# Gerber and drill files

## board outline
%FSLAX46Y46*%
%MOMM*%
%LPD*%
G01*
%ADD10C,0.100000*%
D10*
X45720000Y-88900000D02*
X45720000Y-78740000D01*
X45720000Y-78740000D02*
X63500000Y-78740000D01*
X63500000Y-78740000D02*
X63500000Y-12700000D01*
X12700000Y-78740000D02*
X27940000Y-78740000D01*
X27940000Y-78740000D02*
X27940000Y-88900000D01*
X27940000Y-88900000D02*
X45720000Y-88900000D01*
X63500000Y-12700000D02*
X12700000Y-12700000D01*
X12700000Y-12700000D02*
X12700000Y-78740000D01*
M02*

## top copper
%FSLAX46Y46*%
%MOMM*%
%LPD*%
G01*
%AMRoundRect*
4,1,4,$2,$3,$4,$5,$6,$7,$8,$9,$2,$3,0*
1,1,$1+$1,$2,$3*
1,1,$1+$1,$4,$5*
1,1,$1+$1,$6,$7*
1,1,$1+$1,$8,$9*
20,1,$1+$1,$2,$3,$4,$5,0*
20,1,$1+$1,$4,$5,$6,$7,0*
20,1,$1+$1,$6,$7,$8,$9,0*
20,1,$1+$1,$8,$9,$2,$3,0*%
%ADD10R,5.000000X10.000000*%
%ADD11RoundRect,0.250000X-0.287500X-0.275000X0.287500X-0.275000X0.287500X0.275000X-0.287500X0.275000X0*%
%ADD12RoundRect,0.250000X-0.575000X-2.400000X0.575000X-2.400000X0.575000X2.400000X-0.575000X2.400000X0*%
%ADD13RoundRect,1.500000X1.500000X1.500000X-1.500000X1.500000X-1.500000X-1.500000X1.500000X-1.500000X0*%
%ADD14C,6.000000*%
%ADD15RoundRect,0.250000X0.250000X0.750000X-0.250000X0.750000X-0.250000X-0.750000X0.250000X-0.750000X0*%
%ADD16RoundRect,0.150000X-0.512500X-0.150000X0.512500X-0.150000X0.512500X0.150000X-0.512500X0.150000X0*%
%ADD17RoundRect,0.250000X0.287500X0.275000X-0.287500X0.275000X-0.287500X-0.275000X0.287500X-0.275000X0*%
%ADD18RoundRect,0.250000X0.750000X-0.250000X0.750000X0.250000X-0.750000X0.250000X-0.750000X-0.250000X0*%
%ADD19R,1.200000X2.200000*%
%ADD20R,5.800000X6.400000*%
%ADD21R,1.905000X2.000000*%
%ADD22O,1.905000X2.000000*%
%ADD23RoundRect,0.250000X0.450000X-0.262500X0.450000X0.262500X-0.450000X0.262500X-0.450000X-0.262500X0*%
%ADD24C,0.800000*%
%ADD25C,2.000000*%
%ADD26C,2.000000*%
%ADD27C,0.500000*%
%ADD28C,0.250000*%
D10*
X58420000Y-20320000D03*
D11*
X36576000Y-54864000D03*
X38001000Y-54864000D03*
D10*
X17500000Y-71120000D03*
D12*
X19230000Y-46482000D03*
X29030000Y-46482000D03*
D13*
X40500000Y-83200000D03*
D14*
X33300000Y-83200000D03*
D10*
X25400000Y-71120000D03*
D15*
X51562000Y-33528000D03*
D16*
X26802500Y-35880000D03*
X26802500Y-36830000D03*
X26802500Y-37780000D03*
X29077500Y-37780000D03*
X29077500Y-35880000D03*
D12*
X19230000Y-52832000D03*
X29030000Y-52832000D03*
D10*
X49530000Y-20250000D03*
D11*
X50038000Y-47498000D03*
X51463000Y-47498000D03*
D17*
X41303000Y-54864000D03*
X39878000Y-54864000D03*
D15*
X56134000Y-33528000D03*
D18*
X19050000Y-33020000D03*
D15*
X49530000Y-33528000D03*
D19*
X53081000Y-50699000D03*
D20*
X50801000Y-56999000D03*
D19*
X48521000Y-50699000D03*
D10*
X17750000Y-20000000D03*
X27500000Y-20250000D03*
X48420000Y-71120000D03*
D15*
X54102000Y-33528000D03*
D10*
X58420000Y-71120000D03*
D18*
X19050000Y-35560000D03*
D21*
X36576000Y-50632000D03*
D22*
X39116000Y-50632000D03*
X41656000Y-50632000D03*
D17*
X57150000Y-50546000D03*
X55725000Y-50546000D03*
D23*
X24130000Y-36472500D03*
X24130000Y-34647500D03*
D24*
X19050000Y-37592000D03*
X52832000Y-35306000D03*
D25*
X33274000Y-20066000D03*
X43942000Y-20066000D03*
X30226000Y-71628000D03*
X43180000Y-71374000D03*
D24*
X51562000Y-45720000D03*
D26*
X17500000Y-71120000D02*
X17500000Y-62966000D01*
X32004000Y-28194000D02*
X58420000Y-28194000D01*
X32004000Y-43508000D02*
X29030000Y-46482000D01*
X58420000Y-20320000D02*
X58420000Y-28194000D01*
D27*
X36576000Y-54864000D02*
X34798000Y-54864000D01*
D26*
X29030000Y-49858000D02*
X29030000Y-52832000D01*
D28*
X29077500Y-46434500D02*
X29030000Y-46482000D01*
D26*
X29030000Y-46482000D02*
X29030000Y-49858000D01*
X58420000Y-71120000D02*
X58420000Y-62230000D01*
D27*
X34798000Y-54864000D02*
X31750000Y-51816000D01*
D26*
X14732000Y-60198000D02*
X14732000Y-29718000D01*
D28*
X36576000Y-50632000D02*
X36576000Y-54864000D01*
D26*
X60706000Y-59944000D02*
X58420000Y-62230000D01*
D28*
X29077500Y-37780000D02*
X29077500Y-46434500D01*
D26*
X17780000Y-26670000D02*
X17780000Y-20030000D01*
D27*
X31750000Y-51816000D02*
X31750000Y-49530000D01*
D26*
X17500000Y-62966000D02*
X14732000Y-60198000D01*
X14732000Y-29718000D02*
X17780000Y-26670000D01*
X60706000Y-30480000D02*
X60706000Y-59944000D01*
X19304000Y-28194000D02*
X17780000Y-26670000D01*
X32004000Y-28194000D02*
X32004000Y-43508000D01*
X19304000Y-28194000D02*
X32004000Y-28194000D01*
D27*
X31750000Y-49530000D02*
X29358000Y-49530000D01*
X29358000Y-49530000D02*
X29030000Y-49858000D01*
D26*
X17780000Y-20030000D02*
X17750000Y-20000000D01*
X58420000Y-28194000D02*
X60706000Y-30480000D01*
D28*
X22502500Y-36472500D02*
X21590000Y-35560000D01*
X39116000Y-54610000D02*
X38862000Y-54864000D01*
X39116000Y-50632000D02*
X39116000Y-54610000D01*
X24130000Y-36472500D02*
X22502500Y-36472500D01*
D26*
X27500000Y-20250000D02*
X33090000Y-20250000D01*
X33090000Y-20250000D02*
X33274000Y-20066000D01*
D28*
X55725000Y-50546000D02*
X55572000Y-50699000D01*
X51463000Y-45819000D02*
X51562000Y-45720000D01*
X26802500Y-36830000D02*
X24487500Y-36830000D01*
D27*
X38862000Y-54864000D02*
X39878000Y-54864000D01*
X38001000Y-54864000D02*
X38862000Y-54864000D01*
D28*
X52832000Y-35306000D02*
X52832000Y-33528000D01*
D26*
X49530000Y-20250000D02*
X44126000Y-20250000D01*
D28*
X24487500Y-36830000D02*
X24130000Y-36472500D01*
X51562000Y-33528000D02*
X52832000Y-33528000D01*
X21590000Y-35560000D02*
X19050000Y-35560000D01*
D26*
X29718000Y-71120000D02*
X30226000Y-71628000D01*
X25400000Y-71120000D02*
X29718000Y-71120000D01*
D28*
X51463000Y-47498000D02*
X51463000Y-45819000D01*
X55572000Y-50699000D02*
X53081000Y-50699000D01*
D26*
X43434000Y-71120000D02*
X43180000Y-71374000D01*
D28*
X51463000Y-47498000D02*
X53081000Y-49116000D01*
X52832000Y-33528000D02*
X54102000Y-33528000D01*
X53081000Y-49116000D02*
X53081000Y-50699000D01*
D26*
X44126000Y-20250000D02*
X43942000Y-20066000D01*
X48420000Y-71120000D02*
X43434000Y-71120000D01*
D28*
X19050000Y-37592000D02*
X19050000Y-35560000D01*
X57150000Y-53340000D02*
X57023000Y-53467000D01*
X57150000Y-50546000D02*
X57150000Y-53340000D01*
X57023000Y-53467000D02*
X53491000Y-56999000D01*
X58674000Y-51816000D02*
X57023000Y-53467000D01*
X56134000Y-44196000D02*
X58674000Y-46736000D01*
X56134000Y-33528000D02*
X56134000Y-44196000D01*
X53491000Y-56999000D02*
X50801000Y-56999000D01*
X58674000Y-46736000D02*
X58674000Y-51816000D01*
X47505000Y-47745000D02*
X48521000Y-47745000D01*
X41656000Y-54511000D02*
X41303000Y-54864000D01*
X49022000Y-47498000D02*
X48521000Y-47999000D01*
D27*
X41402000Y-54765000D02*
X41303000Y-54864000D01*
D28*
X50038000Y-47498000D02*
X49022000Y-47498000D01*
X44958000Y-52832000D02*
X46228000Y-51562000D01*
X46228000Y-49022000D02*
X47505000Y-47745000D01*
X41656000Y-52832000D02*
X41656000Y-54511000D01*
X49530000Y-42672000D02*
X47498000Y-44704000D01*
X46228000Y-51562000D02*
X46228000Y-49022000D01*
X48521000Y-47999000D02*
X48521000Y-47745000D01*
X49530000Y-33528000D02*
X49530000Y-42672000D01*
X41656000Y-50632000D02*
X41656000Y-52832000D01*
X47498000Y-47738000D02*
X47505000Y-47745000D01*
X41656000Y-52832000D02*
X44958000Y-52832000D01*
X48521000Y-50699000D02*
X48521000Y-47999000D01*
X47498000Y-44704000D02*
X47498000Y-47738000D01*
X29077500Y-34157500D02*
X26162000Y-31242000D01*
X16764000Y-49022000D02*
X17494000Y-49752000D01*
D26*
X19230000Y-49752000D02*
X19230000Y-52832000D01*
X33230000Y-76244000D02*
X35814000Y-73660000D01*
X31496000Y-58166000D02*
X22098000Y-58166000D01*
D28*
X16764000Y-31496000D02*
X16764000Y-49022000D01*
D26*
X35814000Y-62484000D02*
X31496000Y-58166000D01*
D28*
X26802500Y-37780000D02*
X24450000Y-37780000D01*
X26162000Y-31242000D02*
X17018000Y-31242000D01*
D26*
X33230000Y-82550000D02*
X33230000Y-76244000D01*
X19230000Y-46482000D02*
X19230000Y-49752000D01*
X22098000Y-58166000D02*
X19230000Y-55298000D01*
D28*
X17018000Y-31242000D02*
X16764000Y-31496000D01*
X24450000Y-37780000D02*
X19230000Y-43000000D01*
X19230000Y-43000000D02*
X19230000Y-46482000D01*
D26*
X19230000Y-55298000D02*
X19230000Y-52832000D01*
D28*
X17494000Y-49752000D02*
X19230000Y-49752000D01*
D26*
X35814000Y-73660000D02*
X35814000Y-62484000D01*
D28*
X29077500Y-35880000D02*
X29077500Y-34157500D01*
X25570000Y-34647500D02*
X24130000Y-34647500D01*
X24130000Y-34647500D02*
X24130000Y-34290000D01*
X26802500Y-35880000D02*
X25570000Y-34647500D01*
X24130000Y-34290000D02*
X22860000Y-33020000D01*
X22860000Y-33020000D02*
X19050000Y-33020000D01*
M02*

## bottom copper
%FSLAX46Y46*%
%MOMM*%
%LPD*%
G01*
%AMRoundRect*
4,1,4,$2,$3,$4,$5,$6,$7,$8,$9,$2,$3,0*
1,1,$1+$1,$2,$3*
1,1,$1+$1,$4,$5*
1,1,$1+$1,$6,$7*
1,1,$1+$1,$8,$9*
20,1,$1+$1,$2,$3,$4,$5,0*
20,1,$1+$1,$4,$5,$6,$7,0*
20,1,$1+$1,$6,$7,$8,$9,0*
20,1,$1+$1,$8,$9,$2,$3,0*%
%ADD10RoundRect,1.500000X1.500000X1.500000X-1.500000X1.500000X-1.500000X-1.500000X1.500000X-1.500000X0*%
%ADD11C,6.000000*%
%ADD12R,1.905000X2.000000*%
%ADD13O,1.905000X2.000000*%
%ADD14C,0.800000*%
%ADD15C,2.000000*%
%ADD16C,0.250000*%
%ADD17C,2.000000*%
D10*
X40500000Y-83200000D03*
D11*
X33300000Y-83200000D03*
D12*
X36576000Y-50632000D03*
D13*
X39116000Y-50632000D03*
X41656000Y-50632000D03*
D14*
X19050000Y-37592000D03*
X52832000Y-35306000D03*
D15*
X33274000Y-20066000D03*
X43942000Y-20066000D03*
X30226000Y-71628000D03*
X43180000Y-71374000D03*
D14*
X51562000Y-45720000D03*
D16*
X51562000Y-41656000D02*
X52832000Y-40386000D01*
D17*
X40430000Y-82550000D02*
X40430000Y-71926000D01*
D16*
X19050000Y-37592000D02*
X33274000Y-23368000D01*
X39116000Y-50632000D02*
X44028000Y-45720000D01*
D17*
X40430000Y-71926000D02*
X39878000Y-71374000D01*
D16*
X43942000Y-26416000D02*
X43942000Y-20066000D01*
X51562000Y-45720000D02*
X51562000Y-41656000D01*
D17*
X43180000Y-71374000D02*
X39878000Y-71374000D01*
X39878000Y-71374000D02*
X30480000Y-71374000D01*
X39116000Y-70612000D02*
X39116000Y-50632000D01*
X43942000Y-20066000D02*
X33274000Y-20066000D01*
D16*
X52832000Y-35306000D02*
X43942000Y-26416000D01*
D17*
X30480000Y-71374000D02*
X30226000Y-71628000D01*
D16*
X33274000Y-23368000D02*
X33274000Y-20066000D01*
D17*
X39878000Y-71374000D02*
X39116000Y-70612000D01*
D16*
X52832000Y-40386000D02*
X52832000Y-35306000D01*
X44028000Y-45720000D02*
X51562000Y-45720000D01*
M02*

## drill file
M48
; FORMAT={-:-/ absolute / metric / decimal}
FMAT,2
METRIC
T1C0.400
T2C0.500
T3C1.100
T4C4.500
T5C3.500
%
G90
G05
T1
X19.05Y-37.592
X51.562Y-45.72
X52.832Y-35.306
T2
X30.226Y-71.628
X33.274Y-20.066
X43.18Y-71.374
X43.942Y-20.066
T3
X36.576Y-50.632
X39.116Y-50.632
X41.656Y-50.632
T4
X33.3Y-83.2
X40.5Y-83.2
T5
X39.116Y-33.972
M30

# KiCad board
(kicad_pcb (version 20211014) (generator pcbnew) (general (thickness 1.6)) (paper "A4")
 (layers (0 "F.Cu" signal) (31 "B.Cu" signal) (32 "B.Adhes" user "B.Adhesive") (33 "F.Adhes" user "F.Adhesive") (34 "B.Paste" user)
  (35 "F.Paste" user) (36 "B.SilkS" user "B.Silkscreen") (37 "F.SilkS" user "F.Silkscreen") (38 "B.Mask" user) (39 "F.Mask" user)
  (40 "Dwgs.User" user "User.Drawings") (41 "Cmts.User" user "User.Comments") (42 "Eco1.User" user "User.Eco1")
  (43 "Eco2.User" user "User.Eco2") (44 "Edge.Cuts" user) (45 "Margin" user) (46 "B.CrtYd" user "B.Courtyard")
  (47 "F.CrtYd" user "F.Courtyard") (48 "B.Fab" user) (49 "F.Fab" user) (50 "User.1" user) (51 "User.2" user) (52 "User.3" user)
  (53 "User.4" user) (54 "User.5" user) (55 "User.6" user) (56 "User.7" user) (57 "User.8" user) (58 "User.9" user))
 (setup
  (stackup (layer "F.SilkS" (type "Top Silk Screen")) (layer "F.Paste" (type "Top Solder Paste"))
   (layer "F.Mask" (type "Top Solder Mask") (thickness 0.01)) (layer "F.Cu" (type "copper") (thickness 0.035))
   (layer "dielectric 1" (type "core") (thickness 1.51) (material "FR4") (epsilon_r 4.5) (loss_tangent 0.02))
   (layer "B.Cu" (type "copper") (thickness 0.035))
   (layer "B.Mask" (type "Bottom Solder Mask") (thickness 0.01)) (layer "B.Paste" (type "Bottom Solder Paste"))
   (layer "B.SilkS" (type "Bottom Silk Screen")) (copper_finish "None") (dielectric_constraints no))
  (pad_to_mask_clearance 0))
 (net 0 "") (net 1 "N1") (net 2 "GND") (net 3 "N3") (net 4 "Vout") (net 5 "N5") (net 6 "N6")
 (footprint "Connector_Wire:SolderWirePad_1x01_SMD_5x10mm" (layer "F.Cu") (at 58.42 20.32)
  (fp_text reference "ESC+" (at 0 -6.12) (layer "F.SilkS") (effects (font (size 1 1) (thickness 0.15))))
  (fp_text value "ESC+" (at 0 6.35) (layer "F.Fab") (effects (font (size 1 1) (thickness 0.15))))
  (pad "1" smd rect (at 0 0) (size 5 10) (layers "F.Cu" "F.Paste" "F.Mask") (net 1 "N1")))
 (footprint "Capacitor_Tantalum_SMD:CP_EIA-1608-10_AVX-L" (layer "F.Cu") (at 37.2885 54.864)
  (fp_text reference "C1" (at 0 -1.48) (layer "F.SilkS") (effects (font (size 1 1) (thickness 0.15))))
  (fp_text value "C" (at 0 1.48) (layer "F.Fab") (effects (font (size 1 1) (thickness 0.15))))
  (pad "1" smd roundrect (at -0.7125 0) (size 1.075 1.05) (layers "F.Cu" "F.Paste" "F.Mask") (roundrect_rratio 0.238095) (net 1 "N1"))
  (pad "2" smd roundrect (at 0.7125 0) (size 1.075 1.05) (layers "F.Cu" "F.Paste" "F.Mask") (roundrect_rratio 0.238095) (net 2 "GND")))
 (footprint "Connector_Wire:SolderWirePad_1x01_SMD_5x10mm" (layer "F.Cu") (at 17.5 71.12)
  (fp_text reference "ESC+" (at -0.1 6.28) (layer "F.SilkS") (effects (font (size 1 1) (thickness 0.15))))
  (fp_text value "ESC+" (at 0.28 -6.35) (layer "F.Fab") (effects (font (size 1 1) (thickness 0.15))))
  (pad "1" smd rect (at 0 0) (size 5 10) (layers "F.Cu" "F.Paste" "F.Mask") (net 1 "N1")))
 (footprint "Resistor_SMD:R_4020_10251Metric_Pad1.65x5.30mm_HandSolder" (layer "F.Cu") (at 24.13 46.482)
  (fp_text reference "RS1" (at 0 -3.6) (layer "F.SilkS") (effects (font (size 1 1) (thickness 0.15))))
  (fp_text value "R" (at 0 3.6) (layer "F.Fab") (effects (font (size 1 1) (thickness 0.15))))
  (pad "1" smd roundrect (at -4.9 0) (size 1.65 5.3) (layers "F.Cu" "F.Paste" "F.Mask") (roundrect_rratio 0.151515) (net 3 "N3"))
  (pad "2" smd roundrect (at 4.9 0) (size 1.65 5.3) (layers "F.Cu" "F.Paste" "F.Mask") (roundrect_rratio 0.151515) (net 1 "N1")))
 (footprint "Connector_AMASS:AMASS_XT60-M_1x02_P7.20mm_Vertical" (layer "F.Cu") (at 40.5 83.2 180)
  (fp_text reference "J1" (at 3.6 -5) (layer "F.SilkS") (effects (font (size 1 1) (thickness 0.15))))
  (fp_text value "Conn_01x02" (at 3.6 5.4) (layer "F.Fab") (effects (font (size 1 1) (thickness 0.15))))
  (pad "1" thru_hole roundrect (at 0 0 180) (size 6 6) (drill 4.5) (layers *.Cu *.Mask) (roundrect_rratio 0.25) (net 2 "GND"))
  (pad "2" thru_hole circle (at 7.2 0 180) (size 6 6) (drill 4.5) (layers *.Cu *.Mask) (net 3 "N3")))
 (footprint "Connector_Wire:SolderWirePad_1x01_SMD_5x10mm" (layer "F.Cu") (at 25.4 71.12)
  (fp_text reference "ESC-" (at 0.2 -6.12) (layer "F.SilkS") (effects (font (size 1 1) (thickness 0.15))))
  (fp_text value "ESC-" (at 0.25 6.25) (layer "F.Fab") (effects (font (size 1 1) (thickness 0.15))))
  (pad "1" smd rect (at 0 0) (size 5 10) (layers "F.Cu" "F.Paste" "F.Mask") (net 2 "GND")))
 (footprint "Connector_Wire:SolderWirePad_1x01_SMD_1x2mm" (layer "F.Cu") (at 51.562 33.528 180)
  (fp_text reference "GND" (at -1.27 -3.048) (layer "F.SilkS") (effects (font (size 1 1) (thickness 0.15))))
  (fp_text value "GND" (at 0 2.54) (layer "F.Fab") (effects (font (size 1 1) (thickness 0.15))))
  (pad "1" smd roundrect (at 0 0 180) (size 1 2) (layers "F.Cu" "F.Paste" "F.Mask") (roundrect_rratio 0.25) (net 2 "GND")))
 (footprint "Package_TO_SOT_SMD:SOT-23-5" (layer "F.Cu") (at 27.94 36.83)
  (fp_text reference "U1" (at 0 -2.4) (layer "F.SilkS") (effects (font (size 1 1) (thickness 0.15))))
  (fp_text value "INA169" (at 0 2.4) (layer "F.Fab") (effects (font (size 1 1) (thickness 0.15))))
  (pad "1" smd roundrect (at -1.1375 -0.95) (size 1.325 0.6) (layers "F.Cu" "F.Paste" "F.Mask") (roundrect_rratio 0.25) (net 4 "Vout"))
  (pad "2" smd roundrect (at -1.1375 0) (size 1.325 0.6) (layers "F.Cu" "F.Paste" "F.Mask") (roundrect_rratio 0.25) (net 2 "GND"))
  (pad "3" smd roundrect (at -1.1375 0.95) (size 1.325 0.6) (layers "F.Cu" "F.Paste" "F.Mask") (roundrect_rratio 0.25) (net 3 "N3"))
  (pad "4" smd roundrect (at 1.1375 0.95) (size 1.325 0.6) (layers "F.Cu" "F.Paste" "F.Mask") (roundrect_rratio 0.25) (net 1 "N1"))
  (pad "5" smd roundrect (at 1.1375 -0.95) (size 1.325 0.6) (layers "F.Cu" "F.Paste" "F.Mask") (roundrect_rratio 0.25) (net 3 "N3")))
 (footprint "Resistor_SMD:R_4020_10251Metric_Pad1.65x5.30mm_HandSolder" (layer "F.Cu") (at 24.13 52.832)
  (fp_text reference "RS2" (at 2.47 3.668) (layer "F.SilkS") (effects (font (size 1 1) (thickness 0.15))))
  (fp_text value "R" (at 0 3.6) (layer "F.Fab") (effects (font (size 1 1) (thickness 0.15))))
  (pad "1" smd roundrect (at -4.9 0) (size 1.65 5.3) (layers "F.Cu" "F.Paste" "F.Mask") (roundrect_rratio 0.151515) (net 3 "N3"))
  (pad "2" smd roundrect (at 4.9 0) (size 1.65 5.3) (layers "F.Cu" "F.Paste" "F.Mask") (roundrect_rratio 0.151515) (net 1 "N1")))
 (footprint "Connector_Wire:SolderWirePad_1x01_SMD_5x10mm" (layer "F.Cu") (at 49.53 20.25)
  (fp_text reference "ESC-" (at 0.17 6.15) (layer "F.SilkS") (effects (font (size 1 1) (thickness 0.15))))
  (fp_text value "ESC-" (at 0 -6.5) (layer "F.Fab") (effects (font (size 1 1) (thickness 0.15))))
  (pad "1" smd rect (at 0 0) (size 5 10) (layers "F.Cu" "F.Paste" "F.Mask") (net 2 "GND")))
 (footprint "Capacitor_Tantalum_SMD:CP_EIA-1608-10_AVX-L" (layer "F.Cu") (at 50.7505 47.498)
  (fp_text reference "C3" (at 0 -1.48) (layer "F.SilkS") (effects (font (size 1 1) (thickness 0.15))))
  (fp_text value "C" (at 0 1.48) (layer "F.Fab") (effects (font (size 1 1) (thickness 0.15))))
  (pad "1" smd roundrect (at -0.7125 0) (size 1.075 1.05) (layers "F.Cu" "F.Paste" "F.Mask") (roundrect_rratio 0.238095) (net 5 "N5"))
  (pad "2" smd roundrect (at 0.7125 0) (size 1.075 1.05) (layers "F.Cu" "F.Paste" "F.Mask") (roundrect_rratio 0.238095) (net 2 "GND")))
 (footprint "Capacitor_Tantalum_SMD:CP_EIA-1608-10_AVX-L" (layer "F.Cu") (at 40.5905 54.864 180)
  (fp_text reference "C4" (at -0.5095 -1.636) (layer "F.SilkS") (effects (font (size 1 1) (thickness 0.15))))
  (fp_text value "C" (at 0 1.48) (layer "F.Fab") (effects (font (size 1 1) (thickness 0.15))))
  (pad "1" smd roundrect (at -0.7125 0 180) (size 1.075 1.05) (layers "F.Cu" "F.Paste" "F.Mask") (roundrect_rratio 0.238095) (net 5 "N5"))
  (pad "2" smd roundrect (at 0.7125 0 180) (size 1.075 1.05) (layers "F.Cu" "F.Paste" "F.Mask") (roundrect_rratio 0.238095) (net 2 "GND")))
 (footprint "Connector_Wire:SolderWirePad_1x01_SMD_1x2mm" (layer "F.Cu") (at 56.134 33.528 180)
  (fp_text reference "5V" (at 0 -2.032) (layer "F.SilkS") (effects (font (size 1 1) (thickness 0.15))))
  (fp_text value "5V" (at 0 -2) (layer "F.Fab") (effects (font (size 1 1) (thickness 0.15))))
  (pad "1" smd roundrect (at 0 0 180) (size 1 2) (layers "F.Cu" "F.Paste" "F.Mask") (roundrect_rratio 0.25) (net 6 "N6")))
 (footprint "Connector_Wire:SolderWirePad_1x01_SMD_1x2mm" (layer "F.Cu") (at 19.05 33.02 90)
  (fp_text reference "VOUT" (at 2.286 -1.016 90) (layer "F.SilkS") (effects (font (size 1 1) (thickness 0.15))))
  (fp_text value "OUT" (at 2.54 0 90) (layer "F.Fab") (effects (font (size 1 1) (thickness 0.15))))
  (pad "1" smd roundrect (at 0 0 90) (size 1 2) (layers "F.Cu" "F.Paste" "F.Mask") (roundrect_rratio 0.25) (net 4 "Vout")))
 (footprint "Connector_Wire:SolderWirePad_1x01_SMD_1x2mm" (layer "F.Cu") (at 49.53 33.528 180)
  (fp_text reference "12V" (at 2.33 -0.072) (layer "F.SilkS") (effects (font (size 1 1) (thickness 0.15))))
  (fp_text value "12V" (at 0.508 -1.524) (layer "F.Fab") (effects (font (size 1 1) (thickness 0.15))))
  (pad "1" smd roundrect (at 0 0 180) (size 1 2) (layers "F.Cu" "F.Paste" "F.Mask") (roundrect_rratio 0.25) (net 5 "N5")))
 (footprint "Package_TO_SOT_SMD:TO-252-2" (layer "F.Cu") (at 50.801 54.899 -90)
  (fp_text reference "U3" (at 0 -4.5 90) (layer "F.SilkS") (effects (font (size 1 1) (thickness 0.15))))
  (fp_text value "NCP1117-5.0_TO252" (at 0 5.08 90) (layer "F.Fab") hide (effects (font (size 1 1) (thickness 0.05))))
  (pad "" smd rect (at 0.425 1.525 270) (size 3.05 2.75) (layers "F.Paste"))
  (pad "" smd rect (at 3.775 1.525 270) (size 3.05 2.75) (layers "F.Paste"))
  (pad "" smd rect (at 3.775 -1.525 270) (size 3.05 2.75) (layers "F.Paste"))
  (pad "" smd rect (at 0.425 -1.525 270) (size 3.05 2.75) (layers "F.Paste"))
  (pad "1" smd rect (at -4.2 -2.28 270) (size 2.2 1.2) (layers "F.Cu" "F.Paste" "F.Mask") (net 2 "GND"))
  (pad "2" smd rect (at 2.1 0 270) (size 6.4 5.8) (layers "F.Cu" "F.Mask") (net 6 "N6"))
  (pad "3" smd rect (at -4.2 2.28 270) (size 2.2 1.2) (layers "F.Cu" "F.Paste" "F.Mask") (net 5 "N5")))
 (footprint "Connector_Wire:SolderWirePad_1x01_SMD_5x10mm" (layer "F.Cu") (at 17.75 20)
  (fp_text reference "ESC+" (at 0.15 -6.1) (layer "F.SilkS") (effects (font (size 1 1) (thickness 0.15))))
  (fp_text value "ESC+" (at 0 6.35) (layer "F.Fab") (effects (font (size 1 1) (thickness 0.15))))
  (pad "1" smd rect (at 0 0) (size 5 10) (layers "F.Cu" "F.Paste" "F.Mask") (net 1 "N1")))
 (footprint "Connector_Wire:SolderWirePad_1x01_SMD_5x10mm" (layer "F.Cu") (at 27.5 20.25)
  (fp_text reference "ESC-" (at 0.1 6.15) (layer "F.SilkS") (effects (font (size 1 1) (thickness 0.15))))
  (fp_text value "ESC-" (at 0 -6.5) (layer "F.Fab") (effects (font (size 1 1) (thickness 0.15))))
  (pad "1" smd rect (at 0 0) (size 5 10) (layers "F.Cu" "F.Paste" "F.Mask") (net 2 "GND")))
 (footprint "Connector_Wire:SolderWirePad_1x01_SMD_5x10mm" (layer "F.Cu") (at 48.42 71.12)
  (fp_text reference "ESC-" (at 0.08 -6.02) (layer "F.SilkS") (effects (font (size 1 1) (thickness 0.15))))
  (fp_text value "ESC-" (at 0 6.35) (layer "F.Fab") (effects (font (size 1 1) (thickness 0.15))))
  (pad "1" smd rect (at 0 0) (size 5 10) (layers "F.Cu" "F.Paste" "F.Mask") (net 2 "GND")))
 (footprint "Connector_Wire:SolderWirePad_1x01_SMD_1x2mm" (layer "F.Cu") (at 54.102 33.528 180)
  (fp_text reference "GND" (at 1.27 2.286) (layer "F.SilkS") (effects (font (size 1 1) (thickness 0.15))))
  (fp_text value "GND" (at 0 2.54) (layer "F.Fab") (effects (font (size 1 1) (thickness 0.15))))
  (pad "1" smd roundrect (at 0 0 180) (size 1 2) (layers "F.Cu" "F.Paste" "F.Mask") (roundrect_rratio 0.25) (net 2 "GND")))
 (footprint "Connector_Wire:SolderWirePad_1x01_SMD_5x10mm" (layer "F.Cu") (at 58.42 71.12)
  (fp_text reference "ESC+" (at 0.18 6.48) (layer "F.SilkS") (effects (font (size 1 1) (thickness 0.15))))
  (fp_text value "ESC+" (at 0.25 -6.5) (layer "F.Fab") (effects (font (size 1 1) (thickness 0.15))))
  (pad "1" smd rect (at 0 0) (size 5 10) (layers "F.Cu" "F.Paste" "F.Mask") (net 1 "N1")))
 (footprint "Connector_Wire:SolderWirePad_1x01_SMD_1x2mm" (layer "F.Cu") (at 19.05 35.56 90)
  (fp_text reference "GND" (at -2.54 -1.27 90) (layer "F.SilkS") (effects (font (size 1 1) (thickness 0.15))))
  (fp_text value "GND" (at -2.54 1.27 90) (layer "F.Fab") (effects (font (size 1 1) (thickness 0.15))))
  (pad "1" smd roundrect (at 0 0 90) (size 1 2) (layers "F.Cu" "F.Paste" "F.Mask") (roundrect_rratio 0.25) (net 2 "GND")))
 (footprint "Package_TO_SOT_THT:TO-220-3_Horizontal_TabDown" (layer "F.Cu") (at 36.576 50.632)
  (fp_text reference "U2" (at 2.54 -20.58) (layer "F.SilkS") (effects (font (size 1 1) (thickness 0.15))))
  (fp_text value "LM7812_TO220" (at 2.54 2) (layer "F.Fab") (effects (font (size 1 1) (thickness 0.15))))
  (pad "" np_thru_hole oval (at 2.54 -16.66) (size 3.5 3.5) (drill 3.5) (layers *.Cu *.Mask))
  (pad "1" thru_hole rect (at 0 0) (size 1.905 2) (drill 1.1) (layers *.Cu *.Mask) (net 1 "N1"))
  (pad "2" thru_hole oval (at 2.54 0) (size 1.905 2) (drill 1.1) (layers *.Cu *.Mask) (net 2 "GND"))
  (pad "3" thru_hole oval (at 5.08 0) (size 1.905 2) (drill 1.1) (layers *.Cu *.Mask) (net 5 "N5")))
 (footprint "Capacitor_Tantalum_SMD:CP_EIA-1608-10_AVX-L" (layer "F.Cu") (at 56.4375 50.546 180)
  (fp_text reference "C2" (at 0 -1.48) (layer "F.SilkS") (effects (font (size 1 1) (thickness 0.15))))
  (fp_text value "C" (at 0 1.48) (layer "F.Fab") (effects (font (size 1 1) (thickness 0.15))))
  (pad "1" smd roundrect (at -0.7125 0 180) (size 1.075 1.05) (layers "F.Cu" "F.Paste" "F.Mask") (roundrect_rratio 0.238095) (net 6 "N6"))
  (pad "2" smd roundrect (at 0.7125 0 180) (size 1.075 1.05) (layers "F.Cu" "F.Paste" "F.Mask") (roundrect_rratio 0.238095) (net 2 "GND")))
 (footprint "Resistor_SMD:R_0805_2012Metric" (layer "F.Cu") (at 24.13 35.56 90)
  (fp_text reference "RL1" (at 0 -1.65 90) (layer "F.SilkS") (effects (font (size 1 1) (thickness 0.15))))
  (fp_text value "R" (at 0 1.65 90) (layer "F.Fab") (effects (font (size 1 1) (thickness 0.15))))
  (pad "1" smd roundrect (at -0.9125 0 90) (size 1.025 1.4) (layers "F.Cu" "F.Paste" "F.Mask") (roundrect_rratio 0.243902) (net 2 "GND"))
  (pad "2" smd roundrect (at 0.9125 0 90) (size 1.025 1.4) (layers "F.Cu" "F.Paste" "F.Mask") (roundrect_rratio 0.243902) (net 4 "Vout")))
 (gr_line (start 45.72 88.9) (end 45.72 78.74) (layer "Edge.Cuts") (width 0.1))
 (gr_line (start 45.72 78.74) (end 63.5 78.74) (layer "Edge.Cuts") (width 0.1))
 (gr_line (start 63.5 78.74) (end 63.5 12.7) (layer "Edge.Cuts") (width 0.1))
 (gr_line (start 12.7 78.74) (end 27.94 78.74) (layer "Edge.Cuts") (width 0.1))
 (gr_line (start 27.94 78.74) (end 27.94 88.9) (layer "Edge.Cuts") (width 0.1))
 (gr_line (start 27.94 88.9) (end 45.72 88.9) (layer "Edge.Cuts") (width 0.1))
 (gr_line (start 63.5 12.7) (end 12.7 12.7) (layer "Edge.Cuts") (width 0.1))
 (gr_line (start 12.7 12.7) (end 12.7 78.74) (layer "Edge.Cuts") (width 0.1))
 (segment (start 17.5 71.12) (end 17.5 62.966) (width 2) (layer "F.Cu") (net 1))
 (segment (start 32.004 28.194) (end 58.42 28.194) (width 2) (layer "F.Cu") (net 1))
 (segment (start 32.004 43.508) (end 29.03 46.482) (width 2) (layer "F.Cu") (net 1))
 (segment (start 58.42 20.32) (end 58.42 28.194) (width 2) (layer "F.Cu") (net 1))
 (segment (start 36.576 54.864) (end 34.798 54.864) (width 0.5) (layer "F.Cu") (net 1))
 (segment (start 29.03 49.858) (end 29.03 52.832) (width 2) (layer "F.Cu") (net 1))
 (segment (start 29.0775 46.4345) (end 29.03 46.482) (width 0.25) (layer "F.Cu") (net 1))
 (segment (start 29.03 46.482) (end 29.03 49.858) (width 2) (layer "F.Cu") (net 1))
 (segment (start 58.42 71.12) (end 58.42 62.23) (width 2) (layer "F.Cu") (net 1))
 (segment (start 34.798 54.864) (end 31.75 51.816) (width 0.5) (layer "F.Cu") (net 1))
 (segment (start 14.732 60.198) (end 14.732 29.718) (width 2) (layer "F.Cu") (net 1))
 (segment (start 36.576 50.632) (end 36.576 54.864) (width 0.25) (layer "F.Cu") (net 1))
 (segment (start 60.706 59.944) (end 58.42 62.23) (width 2) (layer "F.Cu") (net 1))
 (segment (start 29.0775 37.78) (end 29.0775 46.4345) (width 0.25) (layer "F.Cu") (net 1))
 (segment (start 17.78 26.67) (end 17.78 20.03) (width 2) (layer "F.Cu") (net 1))
 (segment (start 31.75 51.816) (end 31.75 49.53) (width 0.5) (layer "F.Cu") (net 1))
 (segment (start 17.5 62.966) (end 14.732 60.198) (width 2) (layer "F.Cu") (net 1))
 (segment (start 14.732 29.718) (end 17.78 26.67) (width 2) (layer "F.Cu") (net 1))
 (segment (start 60.706 30.48) (end 60.706 59.944) (width 2) (layer "F.Cu") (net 1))
 (segment (start 19.304 28.194) (end 17.78 26.67) (width 2) (layer "F.Cu") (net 1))
 (segment (start 32.004 28.194) (end 32.004 43.508) (width 2) (layer "F.Cu") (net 1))
 (segment (start 19.304 28.194) (end 32.004 28.194) (width 2) (layer "F.Cu") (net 1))
 (segment (start 31.75 49.53) (end 29.358 49.53) (width 0.5) (layer "F.Cu") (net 1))
 (segment (start 29.358 49.53) (end 29.03 49.858) (width 0.5) (layer "F.Cu") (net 1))
 (segment (start 17.78 20.03) (end 17.75 20) (width 2) (layer "F.Cu") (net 1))
 (segment (start 58.42 28.194) (end 60.706 30.48) (width 2) (layer "F.Cu") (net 1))
 (segment (start 22.5025 36.4725) (end 21.59 35.56) (width 0.25) (layer "F.Cu") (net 2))
 (segment (start 39.116 54.61) (end 38.862 54.864) (width 0.25) (layer "F.Cu") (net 2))
 (segment (start 39.116 50.632) (end 39.116 54.61) (width 0.25) (layer "F.Cu") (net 2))
 (segment (start 24.13 36.4725) (end 22.5025 36.4725) (width 0.25) (layer "F.Cu") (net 2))
 (segment (start 27.5 20.25) (end 33.09 20.25) (width 2) (layer "F.Cu") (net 2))
 (segment (start 33.09 20.25) (end 33.274 20.066) (width 2) (layer "F.Cu") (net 2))
 (segment (start 55.725 50.546) (end 55.572 50.699) (width 0.25) (layer "F.Cu") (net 2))
 (segment (start 51.463 45.819) (end 51.562 45.72) (width 0.25) (layer "F.Cu") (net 2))
 (segment (start 26.8025 36.83) (end 24.4875 36.83) (width 0.25) (layer "F.Cu") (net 2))
 (segment (start 38.862 54.864) (end 39.878 54.864) (width 0.5) (layer "F.Cu") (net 2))
 (segment (start 38.001 54.864) (end 38.862 54.864) (width 0.5) (layer "F.Cu") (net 2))
 (segment (start 52.832 35.306) (end 52.832 33.528) (width 0.25) (layer "F.Cu") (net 2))
 (segment (start 49.53 20.25) (end 44.126 20.25) (width 2) (layer "F.Cu") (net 2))
 (segment (start 24.4875 36.83) (end 24.13 36.4725) (width 0.25) (layer "F.Cu") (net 2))
 (segment (start 51.562 33.528) (end 52.832 33.528) (width 0.25) (layer "F.Cu") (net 2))
 (segment (start 21.59 35.56) (end 19.05 35.56) (width 0.25) (layer "F.Cu") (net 2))
 (segment (start 29.718 71.12) (end 30.226 71.628) (width 2) (layer "F.Cu") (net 2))
 (segment (start 25.4 71.12) (end 29.718 71.12) (width 2) (layer "F.Cu") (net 2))
 (segment (start 51.463 47.498) (end 51.463 45.819) (width 0.25) (layer "F.Cu") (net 2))
 (segment (start 55.572 50.699) (end 53.081 50.699) (width 0.25) (layer "F.Cu") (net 2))
 (segment (start 43.434 71.12) (end 43.18 71.374) (width 2) (layer "F.Cu") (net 2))
 (segment (start 51.463 47.498) (end 53.081 49.116) (width 0.25) (layer "F.Cu") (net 2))
 (segment (start 52.832 33.528) (end 54.102 33.528) (width 0.25) (layer "F.Cu") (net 2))
 (segment (start 53.081 49.116) (end 53.081 50.699) (width 0.25) (layer "F.Cu") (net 2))
 (segment (start 44.126 20.25) (end 43.942 20.066) (width 2) (layer "F.Cu") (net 2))
 (segment (start 48.42 71.12) (end 43.434 71.12) (width 2) (layer "F.Cu") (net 2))
 (segment (start 19.05 37.592) (end 19.05 35.56) (width 0.25) (layer "F.Cu") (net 2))
 (via (at 19.05 37.592) (size 0.8) (drill 0.4) (layers "F.Cu" "B.Cu") (free) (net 2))
 (via (at 52.832 35.306) (size 0.8) (drill 0.4) (layers "F.Cu" "B.Cu") (free) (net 2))
 (via (at 33.274 20.066) (size 2) (drill 0.5) (layers "F.Cu" "B.Cu") (free) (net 2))
 (via (at 43.942 20.066) (size 2) (drill 0.5) (layers "F.Cu" "B.Cu") (free) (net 2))
 (via (at 30.226 71.628) (size 2) (drill 0.5) (layers "F.Cu" "B.Cu") (free) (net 2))
 (via (at 43.18 71.374) (size 2) (drill 0.5) (layers "F.Cu" "B.Cu") (free) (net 2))
 (via (at 51.562 45.72) (size 0.8) (drill 0.4) (layers "F.Cu" "B.Cu") (free) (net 2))
 (segment (start 51.562 41.656) (end 52.832 40.386) (width 0.25) (layer "B.Cu") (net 2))
 (segment (start 40.43 82.55) (end 40.43 71.926) (width 2) (layer "B.Cu") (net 2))
 (segment (start 19.05 37.592) (end 33.274 23.368) (width 0.25) (layer "B.Cu") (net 2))
 (segment (start 39.116 50.632) (end 44.028 45.72) (width 0.25) (layer "B.Cu") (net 2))
 (segment (start 40.43 71.926) (end 39.878 71.374) (width 2) (layer "B.Cu") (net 2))
 (segment (start 43.942 26.416) (end 43.942 20.066) (width 0.25) (layer "B.Cu") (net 2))
 (segment (start 51.562 45.72) (end 51.562 41.656) (width 0.25) (layer "B.Cu") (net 2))
 (segment (start 43.18 71.374) (end 39.878 71.374) (width 2) (layer "B.Cu") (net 2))
 (segment (start 39.878 71.374) (end 30.48 71.374) (width 2) (layer "B.Cu") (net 2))
 (segment (start 39.116 70.612) (end 39.116 50.632) (width 2) (layer "B.Cu") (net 2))
 (segment (start 43.942 20.066) (end 33.274 20.066) (width 2) (layer "B.Cu") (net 2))
 (segment (start 52.832 35.306) (end 43.942 26.416) (width 0.25) (layer "B.Cu") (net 2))
 (segment (start 30.48 71.374) (end 30.226 71.628) (width 2) (layer "B.Cu") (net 2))
 (segment (start 33.274 23.368) (end 33.274 20.066) (width 0.25) (layer "B.Cu") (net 2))
 (segment (start 39.878 71.374) (end 39.116 70.612) (width 2) (layer "B.Cu") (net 2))
 (segment (start 52.832 40.386) (end 52.832 35.306) (width 0.25) (layer "B.Cu") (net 2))
 (segment (start 44.028 45.72) (end 51.562 45.72) (width 0.25) (layer "B.Cu") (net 2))
 (segment (start 57.15 53.34) (end 57.023 53.467) (width 0.25) (layer "F.Cu") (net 6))
 (segment (start 57.15 50.546) (end 57.15 53.34) (width 0.25) (layer "F.Cu") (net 6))
 (segment (start 57.023 53.467) (end 53.491 56.999) (width 0.25) (layer "F.Cu") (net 6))
 (segment (start 58.674 51.816) (end 57.023 53.467) (width 0.25) (layer "F.Cu") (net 6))
 (segment (start 56.134 44.196) (end 58.674 46.736) (width 0.25) (layer "F.Cu") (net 6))
 (segment (start 56.134 33.528) (end 56.134 44.196) (width 0.25) (layer "F.Cu") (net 6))
 (segment (start 53.491 56.999) (end 50.801 56.999) (width 0.25) (layer "F.Cu") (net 6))
 (segment (start 58.674 46.736) (end 58.674 51.816) (width 0.25) (layer "F.Cu") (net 6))
 (segment (start 47.505 47.745) (end 48.521 47.745) (width 0.25) (layer "F.Cu") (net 5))
 (segment (start 41.656 54.511) (end 41.303 54.864) (width 0.25) (layer "F.Cu") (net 5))
 (segment (start 49.022 47.498) (end 48.521 47.999) (width 0.25) (layer "F.Cu") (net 5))
 (segment (start 41.402 54.765) (end 41.303 54.864) (width 0.5) (layer "F.Cu") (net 5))
 (segment (start 50.038 47.498) (end 49.022 47.498) (width 0.25) (layer "F.Cu") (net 5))
 (segment (start 44.958 52.832) (end 46.228 51.562) (width 0.25) (layer "F.Cu") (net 5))
 (segment (start 46.228 49.022) (end 47.505 47.745) (width 0.25) (layer "F.Cu") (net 5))
 (segment (start 41.656 52.832) (end 41.656 54.511) (width 0.25) (layer "F.Cu") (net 5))
 (segment (start 49.53 42.672) (end 47.498 44.704) (width 0.25) (layer "F.Cu") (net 5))
 (segment (start 46.228 51.562) (end 46.228 49.022) (width 0.25) (layer "F.Cu") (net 5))
 (segment (start 48.521 47.999) (end 48.521 47.745) (width 0.25) (layer "F.Cu") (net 5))
 (segment (start 49.53 33.528) (end 49.53 42.672) (width 0.25) (layer "F.Cu") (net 5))
 (segment (start 41.656 50.632) (end 41.656 52.832) (width 0.25) (layer "F.Cu") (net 5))
 (segment (start 47.498 47.738) (end 47.505 47.745) (width 0.25) (layer "F.Cu") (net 5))
 (segment (start 41.656 52.832) (end 44.958 52.832) (width 0.25) (layer "F.Cu") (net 5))
 (segment (start 48.521 50.699) (end 48.521 47.999) (width 0.25) (layer "F.Cu") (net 5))
 (segment (start 47.498 44.704) (end 47.498 47.738) (width 0.25) (layer "F.Cu") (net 5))
 (segment (start 29.0775 34.1575) (end 26.162 31.242) (width 0.25) (layer "F.Cu") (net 3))
 (segment (start 16.764 49.022) (end 17.494 49.752) (width 0.25) (layer "F.Cu") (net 3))
 (segment (start 19.23 49.752) (end 19.23 52.832) (width 2) (layer "F.Cu") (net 3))
 (segment (start 33.23 76.244) (end 35.814 73.66) (width 2) (layer "F.Cu") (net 3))
 (segment (start 31.496 58.166) (end 22.098 58.166) (width 2) (layer "F.Cu") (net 3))
 (segment (start 16.764 31.496) (end 16.764 49.022) (width 0.25) (layer "F.Cu") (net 3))
 (segment (start 35.814 62.484) (end 31.496 58.166) (width 2) (layer "F.Cu") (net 3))
 (segment (start 26.8025 37.78) (end 24.45 37.78) (width 0.25) (layer "F.Cu") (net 3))
 (segment (start 26.162 31.242) (end 17.018 31.242) (width 0.25) (layer "F.Cu") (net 3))
 (segment (start 33.23 82.55) (end 33.23 76.244) (width 2) (layer "F.Cu") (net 3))
 (segment (start 19.23 46.482) (end 19.23 49.752) (width 2) (layer "F.Cu") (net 3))
 (segment (start 22.098 58.166) (end 19.23 55.298) (width 2) (layer "F.Cu") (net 3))
 (segment (start 17.018 31.242) (end 16.764 31.496) (width 0.25) (layer "F.Cu") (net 3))
 (segment (start 24.45 37.78) (end 19.23 43) (width 0.25) (layer "F.Cu") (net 3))
 (segment (start 19.23 43) (end 19.23 46.482) (width 0.25) (layer "F.Cu") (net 3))
 (segment (start 19.23 55.298) (end 19.23 52.832) (width 2) (layer "F.Cu") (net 3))
 (segment (start 17.494 49.752) (end 19.23 49.752) (width 0.25) (layer "F.Cu") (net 3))
 (segment (start 35.814 73.66) (end 35.814 62.484) (width 2) (layer "F.Cu") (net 3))
 (segment (start 29.0775 35.88) (end 29.0775 34.1575) (width 0.25) (layer "F.Cu") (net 3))
 (segment (start 25.57 34.6475) (end 24.13 34.6475) (width 0.25) (layer "F.Cu") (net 4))
 (segment (start 24.13 34.6475) (end 24.13 34.29) (width 0.25) (layer "F.Cu") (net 4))
 (segment (start 26.8025 35.88) (end 25.57 34.6475) (width 0.25) (layer "F.Cu") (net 4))
 (segment (start 24.13 34.29) (end 22.86 33.02) (width 0.25) (layer "F.Cu") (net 4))
 (segment (start 22.86 33.02) (end 19.05 33.02) (width 0.25) (layer "F.Cu") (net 4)))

